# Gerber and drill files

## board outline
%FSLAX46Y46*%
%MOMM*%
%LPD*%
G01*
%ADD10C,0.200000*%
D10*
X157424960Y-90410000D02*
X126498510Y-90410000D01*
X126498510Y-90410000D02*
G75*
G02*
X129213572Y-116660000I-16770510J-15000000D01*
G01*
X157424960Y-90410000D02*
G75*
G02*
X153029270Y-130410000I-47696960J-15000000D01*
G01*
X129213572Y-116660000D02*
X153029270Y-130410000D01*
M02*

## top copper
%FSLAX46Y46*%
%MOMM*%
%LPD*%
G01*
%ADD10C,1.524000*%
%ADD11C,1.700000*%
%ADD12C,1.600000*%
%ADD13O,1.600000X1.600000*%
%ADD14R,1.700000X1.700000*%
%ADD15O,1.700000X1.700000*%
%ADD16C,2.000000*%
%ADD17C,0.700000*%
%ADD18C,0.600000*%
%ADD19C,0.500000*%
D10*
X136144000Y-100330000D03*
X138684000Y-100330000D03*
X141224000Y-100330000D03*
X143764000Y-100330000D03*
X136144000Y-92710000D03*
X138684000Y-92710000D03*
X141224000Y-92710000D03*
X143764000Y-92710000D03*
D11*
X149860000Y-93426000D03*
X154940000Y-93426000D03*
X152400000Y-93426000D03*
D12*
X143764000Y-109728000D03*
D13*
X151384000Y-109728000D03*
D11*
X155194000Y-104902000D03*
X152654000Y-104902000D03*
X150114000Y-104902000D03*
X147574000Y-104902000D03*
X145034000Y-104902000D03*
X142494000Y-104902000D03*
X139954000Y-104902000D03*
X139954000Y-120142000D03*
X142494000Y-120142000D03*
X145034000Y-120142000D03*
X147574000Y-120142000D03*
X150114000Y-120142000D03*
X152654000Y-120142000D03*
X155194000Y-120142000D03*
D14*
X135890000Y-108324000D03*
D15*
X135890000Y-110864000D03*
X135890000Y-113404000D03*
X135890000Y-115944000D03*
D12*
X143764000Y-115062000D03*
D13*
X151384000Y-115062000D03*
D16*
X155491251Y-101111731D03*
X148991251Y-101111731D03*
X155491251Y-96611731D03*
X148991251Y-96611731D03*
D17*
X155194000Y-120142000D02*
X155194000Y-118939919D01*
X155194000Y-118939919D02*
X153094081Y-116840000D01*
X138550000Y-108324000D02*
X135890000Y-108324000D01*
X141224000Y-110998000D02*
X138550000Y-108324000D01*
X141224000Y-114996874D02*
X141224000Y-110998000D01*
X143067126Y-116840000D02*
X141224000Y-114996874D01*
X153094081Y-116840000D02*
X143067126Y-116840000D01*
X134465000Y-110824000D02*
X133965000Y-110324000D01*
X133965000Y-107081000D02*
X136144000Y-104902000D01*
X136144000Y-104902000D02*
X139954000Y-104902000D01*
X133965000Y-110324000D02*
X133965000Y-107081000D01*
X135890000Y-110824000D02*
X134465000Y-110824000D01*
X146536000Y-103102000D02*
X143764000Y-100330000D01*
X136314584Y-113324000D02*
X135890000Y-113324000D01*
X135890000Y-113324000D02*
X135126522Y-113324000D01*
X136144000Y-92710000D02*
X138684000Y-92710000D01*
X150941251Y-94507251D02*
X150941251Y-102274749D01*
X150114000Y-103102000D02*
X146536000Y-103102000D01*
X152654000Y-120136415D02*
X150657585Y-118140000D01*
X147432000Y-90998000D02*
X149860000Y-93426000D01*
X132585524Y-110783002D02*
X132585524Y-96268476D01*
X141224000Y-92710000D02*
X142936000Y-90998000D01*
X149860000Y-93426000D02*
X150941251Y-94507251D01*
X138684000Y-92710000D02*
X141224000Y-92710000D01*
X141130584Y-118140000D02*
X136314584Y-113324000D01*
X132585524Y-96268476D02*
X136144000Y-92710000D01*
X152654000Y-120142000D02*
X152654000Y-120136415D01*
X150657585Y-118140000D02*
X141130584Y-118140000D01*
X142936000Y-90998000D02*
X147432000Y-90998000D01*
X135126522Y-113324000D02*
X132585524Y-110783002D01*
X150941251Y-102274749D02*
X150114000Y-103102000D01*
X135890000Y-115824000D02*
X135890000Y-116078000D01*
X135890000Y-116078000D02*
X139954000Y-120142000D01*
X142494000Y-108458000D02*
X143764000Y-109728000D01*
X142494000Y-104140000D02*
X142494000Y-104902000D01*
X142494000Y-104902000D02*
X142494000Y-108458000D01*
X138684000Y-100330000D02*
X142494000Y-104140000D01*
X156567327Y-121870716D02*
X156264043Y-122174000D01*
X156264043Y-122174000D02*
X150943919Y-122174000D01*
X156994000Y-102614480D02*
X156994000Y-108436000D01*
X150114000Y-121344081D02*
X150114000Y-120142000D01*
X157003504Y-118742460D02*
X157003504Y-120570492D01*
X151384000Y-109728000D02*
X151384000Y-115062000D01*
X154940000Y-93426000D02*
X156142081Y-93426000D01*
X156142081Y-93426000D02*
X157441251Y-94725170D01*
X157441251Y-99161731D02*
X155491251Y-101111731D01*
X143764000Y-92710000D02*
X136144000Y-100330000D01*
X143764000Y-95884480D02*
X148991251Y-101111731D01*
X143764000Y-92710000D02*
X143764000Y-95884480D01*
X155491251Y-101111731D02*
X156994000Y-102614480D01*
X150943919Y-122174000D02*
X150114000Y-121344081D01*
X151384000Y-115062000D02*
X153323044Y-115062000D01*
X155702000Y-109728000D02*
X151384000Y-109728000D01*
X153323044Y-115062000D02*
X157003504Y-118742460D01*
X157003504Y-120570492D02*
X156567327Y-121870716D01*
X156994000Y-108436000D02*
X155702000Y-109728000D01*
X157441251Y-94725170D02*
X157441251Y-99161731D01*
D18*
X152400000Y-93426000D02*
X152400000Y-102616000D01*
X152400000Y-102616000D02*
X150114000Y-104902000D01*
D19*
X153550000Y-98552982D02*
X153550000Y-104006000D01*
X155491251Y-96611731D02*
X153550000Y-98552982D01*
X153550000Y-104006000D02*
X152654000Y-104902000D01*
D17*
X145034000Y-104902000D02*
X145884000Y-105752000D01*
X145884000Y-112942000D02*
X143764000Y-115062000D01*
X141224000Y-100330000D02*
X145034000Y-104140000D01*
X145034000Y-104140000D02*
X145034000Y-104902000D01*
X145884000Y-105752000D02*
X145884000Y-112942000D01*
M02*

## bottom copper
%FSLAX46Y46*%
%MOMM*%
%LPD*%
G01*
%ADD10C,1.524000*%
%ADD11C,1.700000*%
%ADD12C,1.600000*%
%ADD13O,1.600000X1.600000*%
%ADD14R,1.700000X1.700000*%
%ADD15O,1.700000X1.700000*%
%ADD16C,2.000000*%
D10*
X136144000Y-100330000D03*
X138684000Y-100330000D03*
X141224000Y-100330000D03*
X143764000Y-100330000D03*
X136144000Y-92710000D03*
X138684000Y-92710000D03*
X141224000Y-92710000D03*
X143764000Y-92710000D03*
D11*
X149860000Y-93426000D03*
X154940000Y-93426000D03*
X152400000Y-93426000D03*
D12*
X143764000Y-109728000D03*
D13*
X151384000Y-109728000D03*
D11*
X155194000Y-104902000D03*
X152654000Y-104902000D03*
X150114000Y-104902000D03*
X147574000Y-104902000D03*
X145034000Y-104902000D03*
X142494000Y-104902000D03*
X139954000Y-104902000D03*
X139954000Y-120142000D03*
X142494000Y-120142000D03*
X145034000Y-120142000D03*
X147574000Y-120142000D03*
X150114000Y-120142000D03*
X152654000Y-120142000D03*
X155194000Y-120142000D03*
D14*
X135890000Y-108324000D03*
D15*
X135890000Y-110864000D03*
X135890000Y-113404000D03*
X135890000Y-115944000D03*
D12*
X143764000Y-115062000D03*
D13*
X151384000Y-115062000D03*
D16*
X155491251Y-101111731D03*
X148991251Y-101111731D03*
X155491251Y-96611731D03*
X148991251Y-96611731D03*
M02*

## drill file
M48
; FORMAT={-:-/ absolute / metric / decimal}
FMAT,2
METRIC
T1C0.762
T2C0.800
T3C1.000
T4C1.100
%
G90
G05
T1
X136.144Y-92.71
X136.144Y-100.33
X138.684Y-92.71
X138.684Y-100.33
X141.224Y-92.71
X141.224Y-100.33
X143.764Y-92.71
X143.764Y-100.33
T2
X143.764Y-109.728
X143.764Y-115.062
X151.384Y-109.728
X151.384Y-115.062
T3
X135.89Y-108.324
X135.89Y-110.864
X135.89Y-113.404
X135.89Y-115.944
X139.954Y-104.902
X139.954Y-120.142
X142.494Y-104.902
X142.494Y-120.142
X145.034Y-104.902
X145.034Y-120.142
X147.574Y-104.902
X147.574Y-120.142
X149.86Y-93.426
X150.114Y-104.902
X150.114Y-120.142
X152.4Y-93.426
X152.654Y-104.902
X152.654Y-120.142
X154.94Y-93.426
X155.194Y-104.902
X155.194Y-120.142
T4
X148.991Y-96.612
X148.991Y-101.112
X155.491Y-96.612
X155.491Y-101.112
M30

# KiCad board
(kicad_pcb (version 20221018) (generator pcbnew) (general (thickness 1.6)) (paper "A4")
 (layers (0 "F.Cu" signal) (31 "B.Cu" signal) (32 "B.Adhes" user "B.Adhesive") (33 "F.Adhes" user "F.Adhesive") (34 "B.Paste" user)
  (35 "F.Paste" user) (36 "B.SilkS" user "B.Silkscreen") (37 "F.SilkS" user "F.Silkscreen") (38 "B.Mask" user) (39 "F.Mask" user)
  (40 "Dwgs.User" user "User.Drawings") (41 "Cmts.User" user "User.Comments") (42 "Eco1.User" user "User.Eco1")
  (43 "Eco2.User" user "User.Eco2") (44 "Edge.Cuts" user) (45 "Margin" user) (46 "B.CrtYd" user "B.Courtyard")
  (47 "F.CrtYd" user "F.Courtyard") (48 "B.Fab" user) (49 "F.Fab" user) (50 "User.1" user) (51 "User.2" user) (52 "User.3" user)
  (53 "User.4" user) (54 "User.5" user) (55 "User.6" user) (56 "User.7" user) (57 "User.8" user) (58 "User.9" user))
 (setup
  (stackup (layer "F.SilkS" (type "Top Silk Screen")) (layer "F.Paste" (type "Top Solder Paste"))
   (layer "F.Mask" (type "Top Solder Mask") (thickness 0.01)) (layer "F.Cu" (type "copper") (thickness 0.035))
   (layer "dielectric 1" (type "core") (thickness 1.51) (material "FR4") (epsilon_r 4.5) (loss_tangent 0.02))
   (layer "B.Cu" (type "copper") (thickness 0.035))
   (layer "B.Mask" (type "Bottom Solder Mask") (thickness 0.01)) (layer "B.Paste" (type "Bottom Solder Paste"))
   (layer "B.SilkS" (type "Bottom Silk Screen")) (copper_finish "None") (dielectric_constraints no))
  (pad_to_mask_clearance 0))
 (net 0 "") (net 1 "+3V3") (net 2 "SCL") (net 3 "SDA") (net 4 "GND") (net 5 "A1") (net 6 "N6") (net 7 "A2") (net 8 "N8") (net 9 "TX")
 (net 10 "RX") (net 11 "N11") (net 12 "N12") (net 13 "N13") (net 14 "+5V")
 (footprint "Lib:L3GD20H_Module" (layer "F.Cu") (at 141.224 95.25 90)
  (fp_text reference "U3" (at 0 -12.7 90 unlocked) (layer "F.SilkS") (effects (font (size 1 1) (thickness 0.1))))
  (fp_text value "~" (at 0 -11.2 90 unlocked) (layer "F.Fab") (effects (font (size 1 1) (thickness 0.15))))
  (pad "1" thru_hole circle (at -5.08 -5.08 90) (size 1.524 1.524) (drill 0.762) (layers "*.Cu" "*.Mask") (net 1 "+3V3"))
  (pad "2" thru_hole circle (at -5.08 -2.54 90) (size 1.524 1.524) (drill 0.762) (layers "*.Cu" "*.Mask") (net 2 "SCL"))
  (pad "3" thru_hole circle (at -5.08 0 90) (size 1.524 1.524) (drill 0.762) (layers "*.Cu" "*.Mask") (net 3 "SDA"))
  (pad "4" thru_hole circle (at -5.08 2.54 90) (size 1.524 1.524) (drill 0.762) (layers "*.Cu" "*.Mask") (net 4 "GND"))
  (pad "5" thru_hole circle (at 2.54 -5.08 90) (size 1.524 1.524) (drill 0.762) (layers "*.Cu" "*.Mask") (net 4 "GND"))
  (pad "6" thru_hole circle (at 2.54 -2.54 90) (size 1.524 1.524) (drill 0.762) (layers "*.Cu" "*.Mask") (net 4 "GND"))
  (pad "7" thru_hole circle (at 2.54 0 90) (size 1.524 1.524) (drill 0.762) (layers "*.Cu" "*.Mask") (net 4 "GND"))
  (pad "8" thru_hole circle (at 2.54 2.54 90) (size 1.524 1.524) (drill 0.762) (layers "*.Cu" "*.Mask") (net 1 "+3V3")))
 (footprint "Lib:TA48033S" (layer "F.Cu") (at 152.4 90.886)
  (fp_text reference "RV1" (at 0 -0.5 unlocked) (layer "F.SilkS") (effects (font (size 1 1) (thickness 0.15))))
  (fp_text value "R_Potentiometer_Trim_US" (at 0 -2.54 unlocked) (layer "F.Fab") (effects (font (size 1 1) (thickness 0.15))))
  (pad "1" thru_hole circle (at -2.54 2.54) (size 1.7 1.7) (drill 1) (layers "*.Cu" "*.Mask") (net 4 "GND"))
  (pad "2" thru_hole circle (at 2.54 2.54) (size 1.7 1.7) (drill 1) (layers "*.Cu" "*.Mask") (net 1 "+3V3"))
  (pad "3" thru_hole circle (at 0 2.54) (size 1.7 1.7) (drill 1) (layers "*.Cu" "*.Mask") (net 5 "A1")))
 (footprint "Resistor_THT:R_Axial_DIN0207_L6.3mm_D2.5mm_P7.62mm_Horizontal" (layer "F.Cu") (at 143.764 109.728)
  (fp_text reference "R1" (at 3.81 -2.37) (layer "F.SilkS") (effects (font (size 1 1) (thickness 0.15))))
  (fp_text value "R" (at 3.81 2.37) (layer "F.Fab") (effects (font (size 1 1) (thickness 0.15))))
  (pad "1" thru_hole circle (at 0 0) (size 1.6 1.6) (drill 0.8) (layers "*.Cu" "*.Mask") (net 2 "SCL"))
  (pad "2" thru_hole oval (at 7.62 0) (size 1.6 1.6) (drill 0.8) (layers "*.Cu" "*.Mask") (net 1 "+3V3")))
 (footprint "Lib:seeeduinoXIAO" (layer "F.Cu") (at 147.574 112.522 90)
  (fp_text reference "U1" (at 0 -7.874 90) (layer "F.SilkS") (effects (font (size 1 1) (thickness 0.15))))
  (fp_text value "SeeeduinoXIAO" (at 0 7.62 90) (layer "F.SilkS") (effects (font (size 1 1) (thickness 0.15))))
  (pad "1" thru_hole circle (at 7.62 7.62 90) (size 1.7 1.7) (drill 1) (layers "*.Cu" "*.Mask") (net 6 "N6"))
  (pad "2" thru_hole circle (at 7.62 5.08 90) (size 1.7 1.7) (drill 1) (layers "*.Cu" "*.Mask") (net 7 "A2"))
  (pad "3" thru_hole circle (at 7.62 2.54 90) (size 1.7 1.7) (drill 1) (layers "*.Cu" "*.Mask") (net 5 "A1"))
  (pad "4" thru_hole circle (at 7.62 0 90) (size 1.7 1.7) (drill 1) (layers "*.Cu" "*.Mask") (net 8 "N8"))
  (pad "5" thru_hole circle (at 7.62 -2.54 90) (size 1.7 1.7) (drill 1) (layers "*.Cu" "*.Mask") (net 3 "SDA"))
  (pad "6" thru_hole circle (at 7.62 -5.08 90) (size 1.7 1.7) (drill 1) (layers "*.Cu" "*.Mask") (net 2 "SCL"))
  (pad "7" thru_hole circle (at 7.62 -7.62 90) (size 1.7 1.7) (drill 1) (layers "*.Cu" "*.Mask") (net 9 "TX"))
  (pad "8" thru_hole circle (at -7.62 -7.62 90) (size 1.7 1.7) (drill 1) (layers "*.Cu" "*.Mask") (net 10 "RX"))
  (pad "9" thru_hole circle (at -7.62 -5.08 90) (size 1.7 1.7) (drill 1) (layers "*.Cu" "*.Mask") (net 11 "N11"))
  (pad "10" thru_hole circle (at -7.62 -2.54 90) (size 1.7 1.7) (drill 1) (layers "*.Cu" "*.Mask") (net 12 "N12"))
  (pad "11" thru_hole circle (at -7.62 0 90) (size 1.7 1.7) (drill 1) (layers "*.Cu" "*.Mask") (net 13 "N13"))
  (pad "12" thru_hole circle (at -7.62 2.54 90) (size 1.7 1.7) (drill 1) (layers "*.Cu" "*.Mask") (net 1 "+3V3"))
  (pad "13" thru_hole circle (at -7.62 5.08 90) (size 1.7 1.7) (drill 1) (layers "*.Cu" "*.Mask") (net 4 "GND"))
  (pad "14" thru_hole circle (at -7.62 7.62 90) (size 1.7 1.7) (drill 1) (layers "*.Cu" "*.Mask") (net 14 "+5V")))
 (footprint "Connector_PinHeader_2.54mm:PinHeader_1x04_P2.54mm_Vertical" (layer "F.Cu") (at 135.89 108.324)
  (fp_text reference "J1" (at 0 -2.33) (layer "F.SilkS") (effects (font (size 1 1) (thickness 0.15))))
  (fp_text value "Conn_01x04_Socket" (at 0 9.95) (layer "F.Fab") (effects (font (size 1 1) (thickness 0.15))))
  (pad "1" thru_hole rect (at 0 0) (size 1.7 1.7) (drill 1) (layers "*.Cu" "*.Mask") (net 14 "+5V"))
  (pad "2" thru_hole oval (at 0 2.54) (size 1.7 1.7) (drill 1) (layers "*.Cu" "*.Mask") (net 9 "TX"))
  (pad "3" thru_hole oval (at 0 5.08) (size 1.7 1.7) (drill 1) (layers "*.Cu" "*.Mask") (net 4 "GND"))
  (pad "4" thru_hole oval (at 0 7.62) (size 1.7 1.7) (drill 1) (layers "*.Cu" "*.Mask") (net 10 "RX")))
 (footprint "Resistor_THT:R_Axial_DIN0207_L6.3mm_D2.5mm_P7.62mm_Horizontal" (layer "F.Cu") (at 143.764 115.062)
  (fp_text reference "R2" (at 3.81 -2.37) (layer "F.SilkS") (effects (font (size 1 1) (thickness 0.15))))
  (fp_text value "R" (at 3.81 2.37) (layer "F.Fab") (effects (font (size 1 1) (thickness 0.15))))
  (pad "1" thru_hole circle (at 0 0) (size 1.6 1.6) (drill 0.8) (layers "*.Cu" "*.Mask") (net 3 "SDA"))
  (pad "2" thru_hole oval (at 7.62 0) (size 1.6 1.6) (drill 0.8) (layers "*.Cu" "*.Mask") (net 1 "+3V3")))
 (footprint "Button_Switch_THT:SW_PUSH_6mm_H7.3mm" (layer "F.Cu") (at 155.491251 101.111731 180)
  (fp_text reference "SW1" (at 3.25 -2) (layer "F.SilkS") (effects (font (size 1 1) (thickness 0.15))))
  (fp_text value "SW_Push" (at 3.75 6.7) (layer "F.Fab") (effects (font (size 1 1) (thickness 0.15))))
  (pad "1" thru_hole circle (at 0 0 270) (size 2 2) (drill 1.1) (layers "*.Cu" "*.Mask") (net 1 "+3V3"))
  (pad "1" thru_hole circle (at 6.5 0 270) (size 2 2) (drill 1.1) (layers "*.Cu" "*.Mask") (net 1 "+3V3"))
  (pad "2" thru_hole circle (at 0 4.5 270) (size 2 2) (drill 1.1) (layers "*.Cu" "*.Mask") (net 7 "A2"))
  (pad "2" thru_hole circle (at 6.5 4.5 270) (size 2 2) (drill 1.1) (layers "*.Cu" "*.Mask") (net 7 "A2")))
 (gr_line (start 157.42496 90.41) (end 126.49851 90.41) (stroke (width 0.2) (type solid)) (layer "Edge.Cuts"))
 (gr_arc (start 126.49851 90.41) (mid 132.108605 103.095153) (end 129.213572 116.66) (stroke (width 0.2) (type solid)) (layer "Edge.Cuts"))
 (gr_arc (start 157.42496 90.41) (mid 159.4288 110.871733) (end 153.02927 130.41) (stroke (width 0.2) (type solid)) (layer "Edge.Cuts"))
 (gr_line (start 129.213572 116.66) (end 153.02927 130.41) (stroke (width 0.2) (type solid)) (layer "Edge.Cuts"))
 (segment (start 155.194 120.142) (end 155.194 118.939919) (width 0.7) (layer "F.Cu") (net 14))
 (segment (start 155.194 118.939919) (end 153.094081 116.84) (width 0.7) (layer "F.Cu") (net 14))
 (segment (start 138.55 108.324) (end 135.89 108.324) (width 0.7) (layer "F.Cu") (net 14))
 (segment (start 141.224 110.998) (end 138.55 108.324) (width 0.7) (layer "F.Cu") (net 14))
 (segment (start 141.224 114.996874) (end 141.224 110.998) (width 0.7) (layer "F.Cu") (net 14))
 (segment (start 143.067126 116.84) (end 141.224 114.996874) (width 0.7) (layer "F.Cu") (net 14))
 (segment (start 153.094081 116.84) (end 143.067126 116.84) (width 0.7) (layer "F.Cu") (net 14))
 (segment (start 134.465 110.824) (end 133.965 110.324) (width 0.7) (layer "F.Cu") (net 9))
 (segment (start 133.965 107.081) (end 136.144 104.902) (width 0.7) (layer "F.Cu") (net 9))
 (segment (start 136.144 104.902) (end 139.954 104.902) (width 0.7) (layer "F.Cu") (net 9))
 (segment (start 133.965 110.324) (end 133.965 107.081) (width 0.7) (layer "F.Cu") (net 9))
 (segment (start 135.89 110.824) (end 134.465 110.824) (width 0.7) (layer "F.Cu") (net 9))
 (segment (start 146.536 103.102) (end 143.764 100.33) (width 0.7) (layer "F.Cu") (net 4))
 (segment (start 136.314584 113.324) (end 135.89 113.324) (width 0.7) (layer "F.Cu") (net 4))
 (segment (start 135.89 113.324) (end 135.126522 113.324) (width 0.7) (layer "F.Cu") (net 4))
 (segment (start 136.144 92.71) (end 138.684 92.71) (width 0.7) (layer "F.Cu") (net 4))
 (segment (start 150.941251 94.507251) (end 150.941251 102.274749) (width 0.7) (layer "F.Cu") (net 4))
 (segment (start 150.114 103.102) (end 146.536 103.102) (width 0.7) (layer "F.Cu") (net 4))
 (segment (start 152.654 120.136415) (end 150.657585 118.14) (width 0.7) (layer "F.Cu") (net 4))
 (segment (start 147.432 90.998) (end 149.86 93.426) (width 0.7) (layer "F.Cu") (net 4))
 (segment (start 132.585524 110.783002) (end 132.585524 96.268476) (width 0.7) (layer "F.Cu") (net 4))
 (segment (start 141.224 92.71) (end 142.936 90.998) (width 0.7) (layer "F.Cu") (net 4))
 (segment (start 149.86 93.426) (end 150.941251 94.507251) (width 0.7) (layer "F.Cu") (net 4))
 (segment (start 138.684 92.71) (end 141.224 92.71) (width 0.7) (layer "F.Cu") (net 4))
 (segment (start 141.130584 118.14) (end 136.314584 113.324) (width 0.7) (layer "F.Cu") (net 4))
 (segment (start 132.585524 96.268476) (end 136.144 92.71) (width 0.7) (layer "F.Cu") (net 4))
 (segment (start 152.654 120.142) (end 152.654 120.136415) (width 0.7) (layer "F.Cu") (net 4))
 (segment (start 150.657585 118.14) (end 141.130584 118.14) (width 0.7) (layer "F.Cu") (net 4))
 (segment (start 142.936 90.998) (end 147.432 90.998) (width 0.7) (layer "F.Cu") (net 4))
 (segment (start 135.126522 113.324) (end 132.585524 110.783002) (width 0.7) (layer "F.Cu") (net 4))
 (segment (start 150.941251 102.274749) (end 150.114 103.102) (width 0.7) (layer "F.Cu") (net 4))
 (segment (start 135.89 115.824) (end 135.89 116.078) (width 0.7) (layer "F.Cu") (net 10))
 (segment (start 135.89 116.078) (end 139.954 120.142) (width 0.7) (layer "F.Cu") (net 10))
 (segment (start 142.494 108.458) (end 143.764 109.728) (width 0.7) (layer "F.Cu") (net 2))
 (segment (start 142.494 104.14) (end 142.494 104.902) (width 0.7) (layer "F.Cu") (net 2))
 (segment (start 142.494 104.902) (end 142.494 108.458) (width 0.7) (layer "F.Cu") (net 2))
 (segment (start 138.684 100.33) (end 142.494 104.14) (width 0.7) (layer "F.Cu") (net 2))
 (segment (start 156.567327 121.870716) (end 156.264043 122.174) (width 0.7) (layer "F.Cu") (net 1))
 (segment (start 156.264043 122.174) (end 150.943919 122.174) (width 0.7) (layer "F.Cu") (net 1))
 (segment (start 156.994 102.61448) (end 156.994 108.436) (width 0.7) (layer "F.Cu") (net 1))
 (segment (start 150.114 121.344081) (end 150.114 120.142) (width 0.7) (layer "F.Cu") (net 1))
 (segment (start 157.003504 118.74246) (end 157.003504 120.570492) (width 0.7) (layer "F.Cu") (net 1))
 (segment (start 151.384 109.728) (end 151.384 115.062) (width 0.7) (layer "F.Cu") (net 1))
 (segment (start 154.94 93.426) (end 156.142081 93.426) (width 0.7) (layer "F.Cu") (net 1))
 (segment (start 156.142081 93.426) (end 157.441251 94.72517) (width 0.7) (layer "F.Cu") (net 1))
 (segment (start 157.441251 99.161731) (end 155.491251 101.111731) (width 0.7) (layer "F.Cu") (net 1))
 (segment (start 143.764 92.71) (end 136.144 100.33) (width 0.7) (layer "F.Cu") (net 1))
 (segment (start 143.764 95.88448) (end 148.991251 101.111731) (width 0.7) (layer "F.Cu") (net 1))
 (segment (start 143.764 92.71) (end 143.764 95.88448) (width 0.7) (layer "F.Cu") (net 1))
 (segment (start 155.491251 101.111731) (end 156.994 102.61448) (width 0.7) (layer "F.Cu") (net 1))
 (segment (start 150.943919 122.174) (end 150.114 121.344081) (width 0.7) (layer "F.Cu") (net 1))
 (segment (start 151.384 115.062) (end 153.323044 115.062) (width 0.7) (layer "F.Cu") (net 1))
 (segment (start 155.702 109.728) (end 151.384 109.728) (width 0.7) (layer "F.Cu") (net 1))
 (segment (start 153.323044 115.062) (end 157.003504 118.74246) (width 0.7) (layer "F.Cu") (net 1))
 (segment (start 157.003504 120.570492) (end 156.567327 121.870716) (width 0.7) (layer "F.Cu") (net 1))
 (segment (start 156.994 108.436) (end 155.702 109.728) (width 0.7) (layer "F.Cu") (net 1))
 (segment (start 157.441251 94.72517) (end 157.441251 99.161731) (width 0.7) (layer "F.Cu") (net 1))
 (segment (start 152.4 93.426) (end 152.4 102.616) (width 0.6) (layer "F.Cu") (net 5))
 (segment (start 152.4 102.616) (end 150.114 104.902) (width 0.6) (layer "F.Cu") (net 5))
 (segment (start 153.55 98.552982) (end 153.55 104.006) (width 0.5) (layer "F.Cu") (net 7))
 (segment (start 155.491251 96.611731) (end 153.55 98.552982) (width 0.5) (layer "F.Cu") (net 7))
 (segment (start 153.55 104.006) (end 152.654 104.902) (width 0.5) (layer "F.Cu") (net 7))
 (segment (start 145.034 104.902) (end 145.884 105.752) (width 0.7) (layer "F.Cu") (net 3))
 (segment (start 145.884 112.942) (end 143.764 115.062) (width 0.7) (layer "F.Cu") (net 3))
 (segment (start 141.224 100.33) (end 145.034 104.14) (width 0.7) (layer "F.Cu") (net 3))
 (segment (start 145.034 104.14) (end 145.034 104.902) (width 0.7) (layer "F.Cu") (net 3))
 (segment (start 145.884 105.752) (end 145.884 112.942) (width 0.7) (layer "F.Cu") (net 3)))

